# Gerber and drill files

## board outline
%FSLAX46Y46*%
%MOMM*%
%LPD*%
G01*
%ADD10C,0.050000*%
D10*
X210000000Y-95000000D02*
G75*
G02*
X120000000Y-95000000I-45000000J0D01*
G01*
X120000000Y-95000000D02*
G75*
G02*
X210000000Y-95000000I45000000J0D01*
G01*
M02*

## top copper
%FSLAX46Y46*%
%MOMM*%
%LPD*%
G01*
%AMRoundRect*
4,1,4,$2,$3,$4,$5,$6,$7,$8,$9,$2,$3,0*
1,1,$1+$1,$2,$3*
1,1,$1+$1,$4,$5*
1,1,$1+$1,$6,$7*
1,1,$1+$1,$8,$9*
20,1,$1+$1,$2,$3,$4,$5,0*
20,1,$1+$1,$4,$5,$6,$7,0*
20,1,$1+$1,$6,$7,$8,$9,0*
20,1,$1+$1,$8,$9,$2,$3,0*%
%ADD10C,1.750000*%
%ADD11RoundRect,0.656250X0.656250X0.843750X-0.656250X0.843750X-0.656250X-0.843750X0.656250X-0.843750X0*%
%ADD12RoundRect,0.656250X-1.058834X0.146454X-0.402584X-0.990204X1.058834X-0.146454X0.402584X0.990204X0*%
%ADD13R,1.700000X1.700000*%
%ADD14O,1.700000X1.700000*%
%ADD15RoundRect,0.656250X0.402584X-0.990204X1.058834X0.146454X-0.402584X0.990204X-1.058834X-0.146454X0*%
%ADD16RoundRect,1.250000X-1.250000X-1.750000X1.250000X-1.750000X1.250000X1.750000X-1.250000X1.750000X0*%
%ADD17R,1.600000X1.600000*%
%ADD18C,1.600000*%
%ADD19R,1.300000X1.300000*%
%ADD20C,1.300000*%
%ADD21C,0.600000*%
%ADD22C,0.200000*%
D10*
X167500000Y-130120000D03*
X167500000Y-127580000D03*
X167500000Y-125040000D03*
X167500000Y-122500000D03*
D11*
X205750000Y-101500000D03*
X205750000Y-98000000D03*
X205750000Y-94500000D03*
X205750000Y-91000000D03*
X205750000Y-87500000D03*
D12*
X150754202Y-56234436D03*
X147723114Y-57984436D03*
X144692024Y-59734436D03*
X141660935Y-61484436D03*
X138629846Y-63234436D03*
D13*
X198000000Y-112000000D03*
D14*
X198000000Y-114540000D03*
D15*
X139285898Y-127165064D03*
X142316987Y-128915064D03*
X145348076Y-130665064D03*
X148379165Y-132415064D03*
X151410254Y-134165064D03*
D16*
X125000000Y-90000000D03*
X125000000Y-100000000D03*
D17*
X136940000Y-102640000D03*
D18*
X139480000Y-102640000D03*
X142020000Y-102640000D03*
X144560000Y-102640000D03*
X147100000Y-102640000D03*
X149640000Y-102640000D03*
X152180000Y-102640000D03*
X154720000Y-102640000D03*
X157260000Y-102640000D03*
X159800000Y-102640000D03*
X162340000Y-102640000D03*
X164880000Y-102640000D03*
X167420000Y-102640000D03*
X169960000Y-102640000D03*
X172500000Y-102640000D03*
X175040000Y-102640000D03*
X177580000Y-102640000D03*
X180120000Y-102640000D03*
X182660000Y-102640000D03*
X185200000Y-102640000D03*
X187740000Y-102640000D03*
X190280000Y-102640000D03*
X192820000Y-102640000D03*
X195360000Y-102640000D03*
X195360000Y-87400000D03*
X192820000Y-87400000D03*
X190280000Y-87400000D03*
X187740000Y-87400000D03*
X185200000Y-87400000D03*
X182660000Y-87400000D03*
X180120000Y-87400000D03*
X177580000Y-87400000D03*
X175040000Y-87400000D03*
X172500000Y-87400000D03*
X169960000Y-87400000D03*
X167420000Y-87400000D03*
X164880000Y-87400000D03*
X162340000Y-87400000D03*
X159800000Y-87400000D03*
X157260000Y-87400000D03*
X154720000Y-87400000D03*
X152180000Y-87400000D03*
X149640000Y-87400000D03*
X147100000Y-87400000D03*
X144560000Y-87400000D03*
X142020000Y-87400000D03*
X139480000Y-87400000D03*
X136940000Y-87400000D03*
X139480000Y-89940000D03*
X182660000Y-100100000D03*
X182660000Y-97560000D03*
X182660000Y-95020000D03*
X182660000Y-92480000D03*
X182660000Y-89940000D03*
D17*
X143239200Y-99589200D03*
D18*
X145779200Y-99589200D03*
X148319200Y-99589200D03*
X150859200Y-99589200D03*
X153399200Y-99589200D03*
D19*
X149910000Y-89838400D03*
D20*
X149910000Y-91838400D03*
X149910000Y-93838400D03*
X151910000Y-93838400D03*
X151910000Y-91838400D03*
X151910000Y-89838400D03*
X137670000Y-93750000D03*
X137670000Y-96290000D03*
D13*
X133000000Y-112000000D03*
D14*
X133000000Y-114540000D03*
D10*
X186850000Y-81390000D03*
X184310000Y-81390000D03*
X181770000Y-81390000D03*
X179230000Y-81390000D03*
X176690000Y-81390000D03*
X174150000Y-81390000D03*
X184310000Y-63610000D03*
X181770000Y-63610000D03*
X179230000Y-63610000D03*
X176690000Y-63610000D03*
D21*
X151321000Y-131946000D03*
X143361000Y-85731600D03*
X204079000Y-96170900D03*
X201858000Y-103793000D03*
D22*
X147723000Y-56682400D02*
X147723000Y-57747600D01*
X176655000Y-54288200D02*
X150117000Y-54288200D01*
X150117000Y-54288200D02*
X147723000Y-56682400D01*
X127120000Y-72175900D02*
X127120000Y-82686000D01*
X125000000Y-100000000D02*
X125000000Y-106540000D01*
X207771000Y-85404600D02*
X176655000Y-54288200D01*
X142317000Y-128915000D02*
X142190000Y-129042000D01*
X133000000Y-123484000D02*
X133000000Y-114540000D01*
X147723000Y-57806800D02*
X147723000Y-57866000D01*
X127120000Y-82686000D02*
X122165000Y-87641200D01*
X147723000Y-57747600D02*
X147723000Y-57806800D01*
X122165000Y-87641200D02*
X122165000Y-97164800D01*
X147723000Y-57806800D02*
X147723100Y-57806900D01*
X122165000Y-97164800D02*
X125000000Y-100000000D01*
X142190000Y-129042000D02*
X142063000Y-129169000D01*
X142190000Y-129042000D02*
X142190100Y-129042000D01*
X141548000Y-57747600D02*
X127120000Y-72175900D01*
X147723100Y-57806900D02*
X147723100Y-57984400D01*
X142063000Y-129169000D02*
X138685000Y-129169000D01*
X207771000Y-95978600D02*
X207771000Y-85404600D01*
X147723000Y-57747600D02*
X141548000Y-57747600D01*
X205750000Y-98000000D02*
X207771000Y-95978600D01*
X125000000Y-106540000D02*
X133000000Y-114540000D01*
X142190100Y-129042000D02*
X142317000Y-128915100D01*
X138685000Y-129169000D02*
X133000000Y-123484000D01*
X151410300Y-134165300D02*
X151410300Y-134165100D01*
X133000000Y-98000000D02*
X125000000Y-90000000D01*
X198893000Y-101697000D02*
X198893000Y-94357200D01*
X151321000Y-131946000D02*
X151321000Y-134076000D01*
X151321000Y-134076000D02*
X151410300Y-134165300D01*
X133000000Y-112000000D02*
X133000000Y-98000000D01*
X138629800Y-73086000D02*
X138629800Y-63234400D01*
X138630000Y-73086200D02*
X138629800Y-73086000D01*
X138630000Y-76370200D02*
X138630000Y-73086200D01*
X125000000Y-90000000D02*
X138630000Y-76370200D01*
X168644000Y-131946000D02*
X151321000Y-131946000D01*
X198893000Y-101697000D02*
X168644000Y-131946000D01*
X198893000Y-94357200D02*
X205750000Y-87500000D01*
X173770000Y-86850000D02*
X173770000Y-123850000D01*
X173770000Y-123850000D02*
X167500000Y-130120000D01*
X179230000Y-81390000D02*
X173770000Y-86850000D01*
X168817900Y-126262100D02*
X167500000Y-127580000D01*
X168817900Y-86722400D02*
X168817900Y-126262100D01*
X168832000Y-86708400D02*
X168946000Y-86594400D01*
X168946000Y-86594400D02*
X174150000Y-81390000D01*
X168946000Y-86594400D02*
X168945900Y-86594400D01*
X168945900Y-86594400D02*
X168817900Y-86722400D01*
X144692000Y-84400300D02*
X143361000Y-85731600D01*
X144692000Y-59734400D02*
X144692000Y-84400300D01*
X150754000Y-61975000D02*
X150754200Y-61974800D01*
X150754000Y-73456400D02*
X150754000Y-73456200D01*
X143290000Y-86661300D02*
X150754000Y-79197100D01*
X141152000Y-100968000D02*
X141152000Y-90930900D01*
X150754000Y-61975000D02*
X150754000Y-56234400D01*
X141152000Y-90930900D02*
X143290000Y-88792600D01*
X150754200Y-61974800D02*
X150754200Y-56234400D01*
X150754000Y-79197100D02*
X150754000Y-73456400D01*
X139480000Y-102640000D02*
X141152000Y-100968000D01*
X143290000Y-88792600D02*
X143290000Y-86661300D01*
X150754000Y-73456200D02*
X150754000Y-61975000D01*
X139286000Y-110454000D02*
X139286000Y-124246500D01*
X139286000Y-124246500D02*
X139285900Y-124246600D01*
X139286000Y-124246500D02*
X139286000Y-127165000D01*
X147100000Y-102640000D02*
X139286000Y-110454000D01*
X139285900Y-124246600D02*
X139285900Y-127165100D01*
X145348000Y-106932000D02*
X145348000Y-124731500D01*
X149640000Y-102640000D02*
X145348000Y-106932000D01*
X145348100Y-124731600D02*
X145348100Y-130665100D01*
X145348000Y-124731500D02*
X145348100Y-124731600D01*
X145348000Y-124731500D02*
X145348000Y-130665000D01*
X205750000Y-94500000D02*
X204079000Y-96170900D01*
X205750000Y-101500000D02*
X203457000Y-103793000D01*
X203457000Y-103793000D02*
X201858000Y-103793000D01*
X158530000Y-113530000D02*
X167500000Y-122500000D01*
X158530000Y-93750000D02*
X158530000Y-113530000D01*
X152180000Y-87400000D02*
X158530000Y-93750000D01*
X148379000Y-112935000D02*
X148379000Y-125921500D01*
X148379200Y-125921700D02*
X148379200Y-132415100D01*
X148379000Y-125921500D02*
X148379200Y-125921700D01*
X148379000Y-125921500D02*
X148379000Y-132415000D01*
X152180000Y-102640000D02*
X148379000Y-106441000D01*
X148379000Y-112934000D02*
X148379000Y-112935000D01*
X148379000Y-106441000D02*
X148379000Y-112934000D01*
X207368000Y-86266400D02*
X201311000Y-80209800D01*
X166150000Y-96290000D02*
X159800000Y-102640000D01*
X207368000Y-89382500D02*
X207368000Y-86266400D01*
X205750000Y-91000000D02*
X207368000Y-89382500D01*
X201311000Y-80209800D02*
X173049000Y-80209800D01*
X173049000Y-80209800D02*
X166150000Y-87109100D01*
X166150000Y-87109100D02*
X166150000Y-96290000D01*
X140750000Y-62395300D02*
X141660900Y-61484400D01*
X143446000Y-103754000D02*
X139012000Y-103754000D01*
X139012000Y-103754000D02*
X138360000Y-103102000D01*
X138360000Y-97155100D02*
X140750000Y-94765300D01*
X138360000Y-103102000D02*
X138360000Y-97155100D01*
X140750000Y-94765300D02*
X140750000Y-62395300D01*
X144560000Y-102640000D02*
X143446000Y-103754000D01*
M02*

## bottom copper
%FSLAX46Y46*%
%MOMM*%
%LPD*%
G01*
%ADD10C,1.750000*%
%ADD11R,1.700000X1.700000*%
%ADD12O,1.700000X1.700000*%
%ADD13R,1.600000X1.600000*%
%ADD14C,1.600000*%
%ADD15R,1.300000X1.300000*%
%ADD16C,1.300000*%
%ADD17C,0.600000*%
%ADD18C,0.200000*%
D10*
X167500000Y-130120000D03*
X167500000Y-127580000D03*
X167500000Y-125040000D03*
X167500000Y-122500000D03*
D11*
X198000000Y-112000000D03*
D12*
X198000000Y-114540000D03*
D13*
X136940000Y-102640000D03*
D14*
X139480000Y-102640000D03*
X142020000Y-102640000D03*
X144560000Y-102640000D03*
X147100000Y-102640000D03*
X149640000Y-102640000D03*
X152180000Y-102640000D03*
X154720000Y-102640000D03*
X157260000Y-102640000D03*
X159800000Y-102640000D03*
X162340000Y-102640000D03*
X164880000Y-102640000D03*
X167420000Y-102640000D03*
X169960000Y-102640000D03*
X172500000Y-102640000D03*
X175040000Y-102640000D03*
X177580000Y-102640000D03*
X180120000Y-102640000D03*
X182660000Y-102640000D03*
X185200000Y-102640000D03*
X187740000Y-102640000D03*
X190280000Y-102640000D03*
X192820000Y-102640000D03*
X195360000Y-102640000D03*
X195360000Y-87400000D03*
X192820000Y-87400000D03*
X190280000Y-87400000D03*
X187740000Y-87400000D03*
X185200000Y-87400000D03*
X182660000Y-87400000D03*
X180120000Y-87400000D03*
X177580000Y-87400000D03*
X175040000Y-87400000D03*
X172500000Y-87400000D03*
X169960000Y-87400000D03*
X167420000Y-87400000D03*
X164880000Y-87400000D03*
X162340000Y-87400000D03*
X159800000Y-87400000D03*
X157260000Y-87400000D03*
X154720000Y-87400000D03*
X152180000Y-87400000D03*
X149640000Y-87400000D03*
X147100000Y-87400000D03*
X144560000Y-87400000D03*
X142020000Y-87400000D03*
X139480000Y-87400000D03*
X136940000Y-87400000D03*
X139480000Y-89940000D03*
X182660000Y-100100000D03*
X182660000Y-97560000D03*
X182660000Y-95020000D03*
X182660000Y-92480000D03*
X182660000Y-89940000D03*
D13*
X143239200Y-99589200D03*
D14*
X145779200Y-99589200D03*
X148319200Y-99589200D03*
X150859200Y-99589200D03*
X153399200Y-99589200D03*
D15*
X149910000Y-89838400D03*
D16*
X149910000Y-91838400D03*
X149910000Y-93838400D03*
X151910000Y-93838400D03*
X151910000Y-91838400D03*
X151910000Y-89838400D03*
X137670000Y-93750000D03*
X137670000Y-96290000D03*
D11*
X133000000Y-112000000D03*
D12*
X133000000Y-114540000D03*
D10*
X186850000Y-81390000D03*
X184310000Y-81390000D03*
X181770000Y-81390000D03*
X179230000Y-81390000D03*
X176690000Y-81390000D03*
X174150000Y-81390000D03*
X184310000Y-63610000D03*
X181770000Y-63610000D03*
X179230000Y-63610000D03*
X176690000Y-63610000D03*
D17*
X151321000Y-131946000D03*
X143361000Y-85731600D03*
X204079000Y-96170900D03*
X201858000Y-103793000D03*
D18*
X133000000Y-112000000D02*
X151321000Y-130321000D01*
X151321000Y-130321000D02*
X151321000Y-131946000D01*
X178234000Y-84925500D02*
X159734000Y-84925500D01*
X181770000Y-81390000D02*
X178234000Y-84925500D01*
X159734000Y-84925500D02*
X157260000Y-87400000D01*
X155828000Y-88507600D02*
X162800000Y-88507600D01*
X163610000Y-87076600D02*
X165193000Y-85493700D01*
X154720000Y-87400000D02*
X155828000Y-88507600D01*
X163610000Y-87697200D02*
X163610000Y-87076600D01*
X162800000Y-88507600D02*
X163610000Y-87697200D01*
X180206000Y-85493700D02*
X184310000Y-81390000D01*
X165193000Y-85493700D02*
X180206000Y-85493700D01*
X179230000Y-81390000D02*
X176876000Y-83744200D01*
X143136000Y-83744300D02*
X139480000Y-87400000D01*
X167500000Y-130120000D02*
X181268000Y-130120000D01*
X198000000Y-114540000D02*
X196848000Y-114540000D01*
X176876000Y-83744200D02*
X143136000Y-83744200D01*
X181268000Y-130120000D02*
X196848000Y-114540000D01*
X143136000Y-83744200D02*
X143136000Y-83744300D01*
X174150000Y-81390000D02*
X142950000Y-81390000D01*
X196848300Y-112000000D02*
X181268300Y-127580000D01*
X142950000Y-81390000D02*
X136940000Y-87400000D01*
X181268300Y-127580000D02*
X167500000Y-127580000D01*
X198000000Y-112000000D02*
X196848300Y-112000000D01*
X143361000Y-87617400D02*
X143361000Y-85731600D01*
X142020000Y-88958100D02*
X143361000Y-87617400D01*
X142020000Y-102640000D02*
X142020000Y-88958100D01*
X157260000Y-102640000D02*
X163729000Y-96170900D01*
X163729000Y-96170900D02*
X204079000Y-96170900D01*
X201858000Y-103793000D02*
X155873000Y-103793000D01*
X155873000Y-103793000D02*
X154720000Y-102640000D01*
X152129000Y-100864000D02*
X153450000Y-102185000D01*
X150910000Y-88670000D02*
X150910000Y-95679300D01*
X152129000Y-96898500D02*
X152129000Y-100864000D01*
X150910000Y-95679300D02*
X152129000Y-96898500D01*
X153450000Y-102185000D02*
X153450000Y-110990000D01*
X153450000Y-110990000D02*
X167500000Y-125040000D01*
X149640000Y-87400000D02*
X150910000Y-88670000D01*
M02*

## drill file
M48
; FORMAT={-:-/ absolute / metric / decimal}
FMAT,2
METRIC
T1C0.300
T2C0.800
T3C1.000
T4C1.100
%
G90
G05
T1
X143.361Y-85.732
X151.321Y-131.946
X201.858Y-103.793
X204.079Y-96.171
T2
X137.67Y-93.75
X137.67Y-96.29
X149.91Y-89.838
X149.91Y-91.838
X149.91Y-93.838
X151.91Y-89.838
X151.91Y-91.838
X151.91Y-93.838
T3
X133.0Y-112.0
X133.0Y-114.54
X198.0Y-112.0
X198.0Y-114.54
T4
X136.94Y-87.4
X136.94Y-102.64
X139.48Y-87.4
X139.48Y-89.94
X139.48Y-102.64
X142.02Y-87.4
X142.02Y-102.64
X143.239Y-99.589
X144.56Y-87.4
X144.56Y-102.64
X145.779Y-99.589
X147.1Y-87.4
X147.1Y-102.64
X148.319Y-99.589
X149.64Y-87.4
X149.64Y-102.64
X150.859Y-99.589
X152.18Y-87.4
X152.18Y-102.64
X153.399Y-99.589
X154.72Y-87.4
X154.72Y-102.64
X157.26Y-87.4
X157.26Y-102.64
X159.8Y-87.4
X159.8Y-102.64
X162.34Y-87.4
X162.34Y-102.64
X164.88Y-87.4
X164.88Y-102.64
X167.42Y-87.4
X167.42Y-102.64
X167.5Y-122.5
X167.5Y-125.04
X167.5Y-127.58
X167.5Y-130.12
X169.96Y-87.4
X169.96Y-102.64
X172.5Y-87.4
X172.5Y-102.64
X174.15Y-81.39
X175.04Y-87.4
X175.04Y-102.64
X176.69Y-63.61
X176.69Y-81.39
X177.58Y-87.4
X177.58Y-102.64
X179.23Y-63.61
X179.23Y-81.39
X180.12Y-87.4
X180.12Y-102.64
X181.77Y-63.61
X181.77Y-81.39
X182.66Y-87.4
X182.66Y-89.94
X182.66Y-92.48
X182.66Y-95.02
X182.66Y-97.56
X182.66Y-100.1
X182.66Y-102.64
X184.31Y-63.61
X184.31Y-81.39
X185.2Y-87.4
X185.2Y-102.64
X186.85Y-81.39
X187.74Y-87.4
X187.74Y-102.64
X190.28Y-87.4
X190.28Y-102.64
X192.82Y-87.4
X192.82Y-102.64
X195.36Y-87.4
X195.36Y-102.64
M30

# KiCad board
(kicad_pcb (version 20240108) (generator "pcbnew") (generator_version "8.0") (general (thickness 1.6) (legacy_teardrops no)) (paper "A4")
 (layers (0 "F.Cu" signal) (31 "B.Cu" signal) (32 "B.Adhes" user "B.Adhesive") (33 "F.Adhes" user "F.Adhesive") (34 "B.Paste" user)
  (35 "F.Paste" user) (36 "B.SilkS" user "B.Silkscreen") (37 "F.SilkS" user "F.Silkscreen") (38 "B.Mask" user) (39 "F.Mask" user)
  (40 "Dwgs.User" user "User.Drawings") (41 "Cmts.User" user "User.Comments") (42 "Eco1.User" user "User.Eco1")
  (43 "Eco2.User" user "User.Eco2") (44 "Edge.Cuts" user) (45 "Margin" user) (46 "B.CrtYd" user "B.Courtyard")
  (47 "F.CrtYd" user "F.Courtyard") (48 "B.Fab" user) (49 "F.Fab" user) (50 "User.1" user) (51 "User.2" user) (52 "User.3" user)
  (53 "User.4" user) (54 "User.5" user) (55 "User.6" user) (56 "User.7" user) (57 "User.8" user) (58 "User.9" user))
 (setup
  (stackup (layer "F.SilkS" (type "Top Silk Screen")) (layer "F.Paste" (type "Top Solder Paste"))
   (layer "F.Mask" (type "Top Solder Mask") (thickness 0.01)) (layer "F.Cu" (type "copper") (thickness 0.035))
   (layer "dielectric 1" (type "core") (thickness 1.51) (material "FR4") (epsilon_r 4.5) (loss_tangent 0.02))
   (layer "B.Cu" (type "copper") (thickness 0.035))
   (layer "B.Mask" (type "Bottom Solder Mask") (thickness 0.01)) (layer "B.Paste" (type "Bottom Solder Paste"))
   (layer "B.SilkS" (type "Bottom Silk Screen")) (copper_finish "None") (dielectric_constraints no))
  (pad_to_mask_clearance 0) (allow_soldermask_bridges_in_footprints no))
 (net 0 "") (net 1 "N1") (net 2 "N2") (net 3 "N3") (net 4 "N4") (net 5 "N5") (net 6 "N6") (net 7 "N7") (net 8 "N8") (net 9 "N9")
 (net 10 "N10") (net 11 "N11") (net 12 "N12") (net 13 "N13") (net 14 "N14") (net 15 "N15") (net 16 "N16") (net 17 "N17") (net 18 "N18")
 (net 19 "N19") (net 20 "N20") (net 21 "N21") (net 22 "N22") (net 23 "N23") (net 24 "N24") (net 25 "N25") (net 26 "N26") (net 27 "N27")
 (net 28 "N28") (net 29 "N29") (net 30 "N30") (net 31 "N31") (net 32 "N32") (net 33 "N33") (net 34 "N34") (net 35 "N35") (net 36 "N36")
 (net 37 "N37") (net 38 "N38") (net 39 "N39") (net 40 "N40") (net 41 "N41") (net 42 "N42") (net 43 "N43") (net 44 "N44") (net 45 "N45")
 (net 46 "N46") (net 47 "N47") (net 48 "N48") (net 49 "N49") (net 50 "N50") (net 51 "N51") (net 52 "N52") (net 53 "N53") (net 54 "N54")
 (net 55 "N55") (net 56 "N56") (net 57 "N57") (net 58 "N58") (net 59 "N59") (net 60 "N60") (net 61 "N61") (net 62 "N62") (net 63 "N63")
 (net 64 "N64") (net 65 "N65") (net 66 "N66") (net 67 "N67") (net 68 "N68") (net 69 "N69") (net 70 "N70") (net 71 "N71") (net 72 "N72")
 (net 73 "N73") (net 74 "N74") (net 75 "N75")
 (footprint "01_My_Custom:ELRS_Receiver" (layer "F.Cu") (at 181.2 126.31)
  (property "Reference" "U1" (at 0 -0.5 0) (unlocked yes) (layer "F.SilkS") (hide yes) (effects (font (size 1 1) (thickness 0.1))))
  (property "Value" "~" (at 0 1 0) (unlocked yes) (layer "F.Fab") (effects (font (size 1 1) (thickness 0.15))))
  (pad "1" thru_hole circle (at -13.7 3.81) (size 1.75 1.75) (drill 1.1) (layers "*.Cu" "*.Mask") (remove_unused_layers no) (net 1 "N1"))
  (pad "2" thru_hole circle (at -13.7 1.27) (size 1.75 1.75) (drill 1.1) (layers "*.Cu" "*.Mask") (remove_unused_layers no) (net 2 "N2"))
  (pad "3" thru_hole circle (at -13.7 -1.27) (size 1.75 1.75) (drill 1.1) (layers "*.Cu" "*.Mask") (remove_unused_layers no) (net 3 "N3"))
  (pad "4" thru_hole circle (at -13.7 -3.81) (size 1.75 1.75) (drill 1.1) (layers "*.Cu" "*.Mask") (remove_unused_layers no) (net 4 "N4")))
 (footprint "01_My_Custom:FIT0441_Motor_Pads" (layer "F.Cu") (at 203.25 97.5 180)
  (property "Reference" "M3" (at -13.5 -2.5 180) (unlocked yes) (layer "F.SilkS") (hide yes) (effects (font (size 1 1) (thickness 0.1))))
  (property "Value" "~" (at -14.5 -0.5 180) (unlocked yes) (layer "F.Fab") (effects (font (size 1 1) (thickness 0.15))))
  (pad "1" smd roundrect (at -2.5 -4 180) (size 2.625 3) (layers "F.Cu" "F.Paste" "F.Mask") (roundrect_rratio 0.25) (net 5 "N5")
   (thermal_bridge_angle 45))
  (pad "2" smd roundrect (at -2.5 -0.5 180) (size 2.625 3) (layers "F.Cu" "F.Paste" "F.Mask") (roundrect_rratio 0.25) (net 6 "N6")
   (thermal_bridge_angle 45))
  (pad "3" smd roundrect (at -2.5 3 180) (size 2.625 3) (layers "F.Cu" "F.Paste" "F.Mask") (roundrect_rratio 0.25) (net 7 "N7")
   (thermal_bridge_angle 45))
  (pad "4" smd roundrect (at -2.5 6.5 180) (size 2.625 3) (layers "F.Cu" "F.Paste" "F.Mask") (roundrect_rratio 0.25) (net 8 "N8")
   (thermal_bridge_angle 45))
  (pad "5" smd roundrect (at -2.5 10 180) (size 2.625 3) (layers "F.Cu" "F.Paste" "F.Mask") (roundrect_rratio 0.25) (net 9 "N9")
   (thermal_bridge_angle 45)))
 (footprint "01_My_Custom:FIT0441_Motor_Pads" (layer "F.Cu") (at 148.5401 60.3995 -60)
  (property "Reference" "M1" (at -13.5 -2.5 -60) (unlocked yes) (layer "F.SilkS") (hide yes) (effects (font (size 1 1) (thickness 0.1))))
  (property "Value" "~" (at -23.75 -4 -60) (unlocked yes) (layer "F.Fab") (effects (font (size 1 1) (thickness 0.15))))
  (pad "1" smd roundrect (at -2.5 -4.000001 300) (size 2.625 3) (layers "F.Cu" "F.Paste" "F.Mask") (roundrect_rratio 0.25) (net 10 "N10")
   (thermal_bridge_angle 45))
  (pad "2" smd roundrect (at -2.5 -0.500001 300) (size 2.625 3) (layers "F.Cu" "F.Paste" "F.Mask") (roundrect_rratio 0.25) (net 6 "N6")
   (thermal_bridge_angle 45))
  (pad "3" smd roundrect (at -2.5 3 300) (size 2.625 3) (layers "F.Cu" "F.Paste" "F.Mask") (roundrect_rratio 0.25) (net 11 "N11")
   (thermal_bridge_angle 45))
  (pad "4" smd roundrect (at -2.5 6.5 300) (size 2.625 3) (layers "F.Cu" "F.Paste" "F.Mask") (roundrect_rratio 0.25) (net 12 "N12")
   (thermal_bridge_angle 45))
  (pad "5" smd roundrect (at -2.5 10 300) (size 2.625 3) (layers "F.Cu" "F.Paste" "F.Mask") (roundrect_rratio 0.25) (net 9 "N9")
   (thermal_bridge_angle 45)))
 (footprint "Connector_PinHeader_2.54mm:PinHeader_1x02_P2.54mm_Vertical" (layer "F.Cu") (at 198 112)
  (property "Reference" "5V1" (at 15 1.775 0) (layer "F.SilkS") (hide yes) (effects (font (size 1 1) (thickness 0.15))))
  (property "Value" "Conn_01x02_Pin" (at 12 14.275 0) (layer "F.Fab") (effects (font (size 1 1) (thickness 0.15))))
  (pad "1" thru_hole rect (at 0 0) (size 1.7 1.7) (drill 1) (layers "*.Cu" "*.Mask") (remove_unused_layers no) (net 2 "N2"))
  (pad "2" thru_hole oval (at 0 2.54) (size 1.7 1.7) (drill 1) (layers "*.Cu" "*.Mask") (remove_unused_layers no) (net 1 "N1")))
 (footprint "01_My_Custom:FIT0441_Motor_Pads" (layer "F.Cu") (at 144 127 60)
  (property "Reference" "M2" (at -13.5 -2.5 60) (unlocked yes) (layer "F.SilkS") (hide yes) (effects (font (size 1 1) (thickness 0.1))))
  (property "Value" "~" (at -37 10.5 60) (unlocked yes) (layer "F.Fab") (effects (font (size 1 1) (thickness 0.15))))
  (pad "1" smd roundrect (at -2.500001 -4 60) (size 2.625 3) (layers "F.Cu" "F.Paste" "F.Mask") (roundrect_rratio 0.25) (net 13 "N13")
   (thermal_bridge_angle 45))
  (pad "2" smd roundrect (at -2.500001 -0.5 60) (size 2.625 3) (layers "F.Cu" "F.Paste" "F.Mask") (roundrect_rratio 0.25) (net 6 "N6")
   (thermal_bridge_angle 45))
  (pad "3" smd roundrect (at -2.500001 3 60) (size 2.625 3) (layers "F.Cu" "F.Paste" "F.Mask") (roundrect_rratio 0.25) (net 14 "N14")
   (thermal_bridge_angle 45))
  (pad "4" smd roundrect (at -2.5 6.5 60) (size 2.625 3) (layers "F.Cu" "F.Paste" "F.Mask") (roundrect_rratio 0.25) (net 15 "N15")
   (thermal_bridge_angle 45))
  (pad "5" smd roundrect (at -2.5 10 60) (size 2.625 3) (layers "F.Cu" "F.Paste" "F.Mask") (roundrect_rratio 0.25) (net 9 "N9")
   (thermal_bridge_angle 45)))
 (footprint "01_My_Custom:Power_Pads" (layer "F.Cu") (at 125 95)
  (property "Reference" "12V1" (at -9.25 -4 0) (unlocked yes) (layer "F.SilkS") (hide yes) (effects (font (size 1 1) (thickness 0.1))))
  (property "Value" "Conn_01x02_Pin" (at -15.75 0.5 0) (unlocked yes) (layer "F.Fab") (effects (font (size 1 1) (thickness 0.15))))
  (pad "1" smd roundrect (at 0 -5) (size 5 6) (layers "F.Cu" "F.Paste" "F.Mask") (roundrect_rratio 0.25) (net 9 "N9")
   (thermal_bridge_angle 45))
  (pad "2" smd roundrect (at 0 5) (size 5 6) (layers "F.Cu" "F.Paste" "F.Mask") (roundrect_rratio 0.25) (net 6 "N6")
   (thermal_bridge_angle 45)))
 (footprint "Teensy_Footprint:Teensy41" (layer "F.Cu") (at 166.15 95.02)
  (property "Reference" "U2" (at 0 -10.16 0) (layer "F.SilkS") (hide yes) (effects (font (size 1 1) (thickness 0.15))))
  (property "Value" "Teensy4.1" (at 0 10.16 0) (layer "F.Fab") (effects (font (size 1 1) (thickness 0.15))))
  (pad "1" thru_hole rect (at -29.21 7.62) (size 1.6 1.6) (drill 1.1) (layers "*.Cu" "*.Mask") (remove_unused_layers no) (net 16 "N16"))
  (pad "2" thru_hole circle (at -26.67 7.62) (size 1.6 1.6) (drill 1.1) (layers "*.Cu" "*.Mask") (remove_unused_layers no) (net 10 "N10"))
  (pad "3" thru_hole circle (at -24.13 7.62) (size 1.6 1.6) (drill 1.1) (layers "*.Cu" "*.Mask") (remove_unused_layers no) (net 11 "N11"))
  (pad "4" thru_hole circle (at -21.59 7.62) (size 1.6 1.6) (drill 1.1) (layers "*.Cu" "*.Mask") (remove_unused_layers no) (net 12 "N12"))
  (pad "5" thru_hole circle (at -19.05 7.62) (size 1.6 1.6) (drill 1.1) (layers "*.Cu" "*.Mask") (remove_unused_layers no) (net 13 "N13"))
  (pad "6" thru_hole circle (at -16.51 7.62) (size 1.6 1.6) (drill 1.1) (layers "*.Cu" "*.Mask") (remove_unused_layers no) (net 14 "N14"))
  (pad "7" thru_hole circle (at -13.97 7.62) (size 1.6 1.6) (drill 1.1) (layers "*.Cu" "*.Mask") (remove_unused_layers no) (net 15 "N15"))
  (pad "8" thru_hole circle (at -11.43 7.62) (size 1.6 1.6) (drill 1.1) (layers "*.Cu" "*.Mask") (remove_unused_layers no) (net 5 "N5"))
  (pad "9" thru_hole circle (at -8.89 7.62) (size 1.6 1.6) (drill 1.1) (layers "*.Cu" "*.Mask") (remove_unused_layers no) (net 7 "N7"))
  (pad "10" thru_hole circle (at -6.35 7.62) (size 1.6 1.6) (drill 1.1) (layers "*.Cu" "*.Mask") (remove_unused_layers no) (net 8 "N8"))
  (pad "11" thru_hole circle (at -3.81 7.62) (size 1.6 1.6) (drill 1.1) (layers "*.Cu" "*.Mask") (remove_unused_layers no) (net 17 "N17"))
  (pad "12" thru_hole circle (at -1.27 7.62) (size 1.6 1.6) (drill 1.1) (layers "*.Cu" "*.Mask") (remove_unused_layers no) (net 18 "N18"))
  (pad "13" thru_hole circle (at 1.27 7.62) (size 1.6 1.6) (drill 1.1) (layers "*.Cu" "*.Mask") (remove_unused_layers no) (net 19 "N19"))
  (pad "14" thru_hole circle (at 3.81 7.62) (size 1.6 1.6) (drill 1.1) (layers "*.Cu" "*.Mask") (remove_unused_layers no) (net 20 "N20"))
  (pad "15" thru_hole circle (at 6.35 7.62) (size 1.6 1.6) (drill 1.1) (layers "*.Cu" "*.Mask") (remove_unused_layers no) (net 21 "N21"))
  (pad "16" thru_hole circle (at 8.89 7.62) (size 1.6 1.6) (drill 1.1) (layers "*.Cu" "*.Mask") (remove_unused_layers no) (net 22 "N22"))
  (pad "17" thru_hole circle (at 11.43 7.62) (size 1.6 1.6) (drill 1.1) (layers "*.Cu" "*.Mask") (remove_unused_layers no) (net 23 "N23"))
  (pad "18" thru_hole circle (at 13.97 7.62) (size 1.6 1.6) (drill 1.1) (layers "*.Cu" "*.Mask") (remove_unused_layers no) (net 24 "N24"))
  (pad "19" thru_hole circle (at 16.51 7.62) (size 1.6 1.6) (drill 1.1) (layers "*.Cu" "*.Mask") (remove_unused_layers no) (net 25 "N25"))
  (pad "20" thru_hole circle (at 19.05 7.62) (size 1.6 1.6) (drill 1.1) (layers "*.Cu" "*.Mask") (remove_unused_layers no) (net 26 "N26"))
  (pad "21" thru_hole circle (at 21.59 7.62) (size 1.6 1.6) (drill 1.1) (layers "*.Cu" "*.Mask") (remove_unused_layers no) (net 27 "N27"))
  (pad "22" thru_hole circle (at 24.13 7.62) (size 1.6 1.6) (drill 1.1) (layers "*.Cu" "*.Mask") (remove_unused_layers no) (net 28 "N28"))
  (pad "23" thru_hole circle (at 26.67 7.62) (size 1.6 1.6) (drill 1.1) (layers "*.Cu" "*.Mask") (remove_unused_layers no) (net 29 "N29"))
  (pad "24" thru_hole circle (at 29.21 7.62) (size 1.6 1.6) (drill 1.1) (layers "*.Cu" "*.Mask") (remove_unused_layers no) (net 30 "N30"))
  (pad "25" thru_hole circle (at 29.21 -7.62) (size 1.6 1.6) (drill 1.1) (layers "*.Cu" "*.Mask") (remove_unused_layers no) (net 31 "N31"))
  (pad "26" thru_hole circle (at 26.67 -7.62) (size 1.6 1.6) (drill 1.1) (layers "*.Cu" "*.Mask") (remove_unused_layers no) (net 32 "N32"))
  (pad "27" thru_hole circle (at 24.13 -7.62) (size 1.6 1.6) (drill 1.1) (layers "*.Cu" "*.Mask") (remove_unused_layers no) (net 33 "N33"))
  (pad "28" thru_hole circle (at 21.59 -7.62) (size 1.6 1.6) (drill 1.1) (layers "*.Cu" "*.Mask") (remove_unused_layers no) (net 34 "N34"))
  (pad "29" thru_hole circle (at 19.05 -7.62) (size 1.6 1.6) (drill 1.1) (layers "*.Cu" "*.Mask") (remove_unused_layers no) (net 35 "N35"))
  (pad "30" thru_hole circle (at 16.51 -7.62) (size 1.6 1.6) (drill 1.1) (layers "*.Cu" "*.Mask") (remove_unused_layers no) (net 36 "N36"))
  (pad "31" thru_hole circle (at 13.97 -7.62) (size 1.6 1.6) (drill 1.1) (layers "*.Cu" "*.Mask") (remove_unused_layers no) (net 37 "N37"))
  (pad "32" thru_hole circle (at 11.43 -7.62) (size 1.6 1.6) (drill 1.1) (layers "*.Cu" "*.Mask") (remove_unused_layers no) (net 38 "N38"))
  (pad "33" thru_hole circle (at 8.89 -7.62) (size 1.6 1.6) (drill 1.1) (layers "*.Cu" "*.Mask") (remove_unused_layers no) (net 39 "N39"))
  (pad "34" thru_hole circle (at 6.35 -7.62) (size 1.6 1.6) (drill 1.1) (layers "*.Cu" "*.Mask") (remove_unused_layers no) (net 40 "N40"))
  (pad "35" thru_hole circle (at 3.81 -7.62) (size 1.6 1.6) (drill 1.1) (layers "*.Cu" "*.Mask") (remove_unused_layers no) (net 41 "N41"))
  (pad "36" thru_hole circle (at 1.27 -7.62) (size 1.6 1.6) (drill 1.1) (layers "*.Cu" "*.Mask") (remove_unused_layers no) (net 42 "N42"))
  (pad "37" thru_hole circle (at -1.27 -7.62) (size 1.6 1.6) (drill 1.1) (layers "*.Cu" "*.Mask") (remove_unused_layers no) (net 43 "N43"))
  (pad "38" thru_hole circle (at -3.81 -7.62) (size 1.6 1.6) (drill 1.1) (layers "*.Cu" "*.Mask") (remove_unused_layers no) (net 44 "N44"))
  (pad "39" thru_hole circle (at -6.35 -7.62) (size 1.6 1.6) (drill 1.1) (layers "*.Cu" "*.Mask") (remove_unused_layers no) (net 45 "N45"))
  (pad "40" thru_hole circle (at -8.89 -7.62) (size 1.6 1.6) (drill 1.1) (layers "*.Cu" "*.Mask") (remove_unused_layers no) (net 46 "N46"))
  (pad "41" thru_hole circle (at -11.43 -7.62) (size 1.6 1.6) (drill 1.1) (layers "*.Cu" "*.Mask") (remove_unused_layers no) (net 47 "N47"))
  (pad "42" thru_hole circle (at -13.97 -7.62) (size 1.6 1.6) (drill 1.1) (layers "*.Cu" "*.Mask") (remove_unused_layers no) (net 4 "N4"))
  (pad "43" thru_hole circle (at -16.51 -7.62) (size 1.6 1.6) (drill 1.1) (layers "*.Cu" "*.Mask") (remove_unused_layers no) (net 3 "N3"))
  (pad "44" thru_hole circle (at -19.05 -7.62) (size 1.6 1.6) (drill 1.1) (layers "*.Cu" "*.Mask") (remove_unused_layers no) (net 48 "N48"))
  (pad "45" thru_hole circle (at -21.59 -7.62) (size 1.6 1.6) (drill 1.1) (layers "*.Cu" "*.Mask") (remove_unused_layers no) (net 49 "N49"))
  (pad "46" thru_hole circle (at -24.13 -7.62) (size 1.6 1.6) (drill 1.1) (layers "*.Cu" "*.Mask") (remove_unused_layers no) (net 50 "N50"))
  (pad "47" thru_hole circle (at -26.67 -7.62) (size 1.6 1.6) (drill 1.1) (layers "*.Cu" "*.Mask") (remove_unused_layers no) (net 1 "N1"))
  (pad "48" thru_hole circle (at -29.21 -7.62) (size 1.6 1.6) (drill 1.1) (layers "*.Cu" "*.Mask") (remove_unused_layers no) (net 2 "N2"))
  (pad "49" thru_hole circle (at -26.67 -5.08) (size 1.6 1.6) (drill 1.1) (layers "*.Cu" "*.Mask") (remove_unused_layers no) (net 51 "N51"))
  (pad "50" thru_hole circle (at 16.51 5.08) (size 1.6 1.6) (drill 1.1) (layers "*.Cu" "*.Mask") (remove_unused_layers no) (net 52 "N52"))
  (pad "51" thru_hole circle (at 16.51 2.54) (size 1.6 1.6) (drill 1.1) (layers "*.Cu" "*.Mask") (remove_unused_layers no) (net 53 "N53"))
  (pad "52" thru_hole circle (at 16.51 0) (size 1.6 1.6) (drill 1.1) (layers "*.Cu" "*.Mask") (remove_unused_layers no) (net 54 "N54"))
  (pad "53" thru_hole circle (at 16.51 -2.54) (size 1.6 1.6) (drill 1.1) (layers "*.Cu" "*.Mask") (remove_unused_layers no) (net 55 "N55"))
  (pad "54" thru_hole circle (at 16.51 -5.08) (size 1.6 1.6) (drill 1.1) (layers "*.Cu" "*.Mask") (remove_unused_layers no) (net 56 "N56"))
  (pad "55" thru_hole rect (at -22.9108 4.5692) (size 1.6 1.6) (drill 1.1) (layers "*.Cu" "*.Mask") (remove_unused_layers no) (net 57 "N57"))
  (pad "56" thru_hole circle (at -20.3708 4.5692) (size 1.6 1.6) (drill 1.1) (layers "*.Cu" "*.Mask") (remove_unused_layers no)
   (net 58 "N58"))
  (pad "57" thru_hole circle (at -17.8308 4.5692) (size 1.6 1.6) (drill 1.1) (layers "*.Cu" "*.Mask") (remove_unused_layers no)
   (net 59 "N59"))
  (pad "58" thru_hole circle (at -15.2908 4.5692) (size 1.6 1.6) (drill 1.1) (layers "*.Cu" "*.Mask") (remove_unused_layers no)
   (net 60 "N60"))
  (pad "59" thru_hole circle (at -12.7508 4.5692) (size 1.6 1.6) (drill 1.1) (layers "*.Cu" "*.Mask") (remove_unused_layers no)
   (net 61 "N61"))
  (pad "60" thru_hole rect (at -16.24 -5.1816) (size 1.3 1.3) (drill 0.8) (layers "*.Cu" "*.Mask") (remove_unused_layers no) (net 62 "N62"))
  (pad "61" thru_hole circle (at -16.24 -3.1816) (size 1.3 1.3) (drill 0.8) (layers "*.Cu" "*.Mask") (remove_unused_layers no)
   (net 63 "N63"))
  (pad "62" thru_hole circle (at -16.24 -1.1816) (size 1.3 1.3) (drill 0.8) (layers "*.Cu" "*.Mask") (remove_unused_layers no)
   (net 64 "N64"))
  (pad "63" thru_hole circle (at -14.24 -1.1816) (size 1.3 1.3) (drill 0.8) (layers "*.Cu" "*.Mask") (remove_unused_layers no)
   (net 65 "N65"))
  (pad "64" thru_hole circle (at -14.24 -3.1816) (size 1.3 1.3) (drill 0.8) (layers "*.Cu" "*.Mask") (remove_unused_layers no)
   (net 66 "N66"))
  (pad "65" thru_hole circle (at -14.24 -5.1816) (size 1.3 1.3) (drill 0.8) (layers "*.Cu" "*.Mask") (remove_unused_layers no)
   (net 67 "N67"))
  (pad "66" thru_hole circle (at -28.48 -1.27) (size 1.3 1.3) (drill 0.8) (layers "*.Cu" "*.Mask") (remove_unused_layers no) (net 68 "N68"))
  (pad "67" thru_hole circle (at -28.48 1.27) (size 1.3 1.3) (drill 0.8) (layers "*.Cu" "*.Mask") (remove_unused_layers no) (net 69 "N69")))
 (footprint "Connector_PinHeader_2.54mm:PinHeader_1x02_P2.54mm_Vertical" (layer "F.Cu") (at 133 112)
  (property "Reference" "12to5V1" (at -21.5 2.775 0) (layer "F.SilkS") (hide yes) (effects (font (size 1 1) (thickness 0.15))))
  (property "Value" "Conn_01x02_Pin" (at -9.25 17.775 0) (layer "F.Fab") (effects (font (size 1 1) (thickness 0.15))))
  (pad "1" thru_hole rect (at 0 0) (size 1.7 1.7) (drill 1) (layers "*.Cu" "*.Mask") (remove_unused_layers no) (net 9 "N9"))
  (pad "2" thru_hole oval (at 0 2.54) (size 1.7 1.7) (drill 1) (layers "*.Cu" "*.Mask") (remove_unused_layers no) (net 6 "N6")))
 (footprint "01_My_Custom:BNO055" (layer "F.Cu") (at 180.5 72.5 -90)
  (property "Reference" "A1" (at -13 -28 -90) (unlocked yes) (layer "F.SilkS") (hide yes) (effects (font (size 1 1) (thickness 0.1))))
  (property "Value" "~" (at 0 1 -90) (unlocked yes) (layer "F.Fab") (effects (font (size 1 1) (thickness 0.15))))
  (pad "1" thru_hole circle (at 8.89 -6.35 270) (size 1.75 1.75) (drill 1.1) (layers "*.Cu" "*.Mask") (remove_unused_layers no)
   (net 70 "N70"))
  (pad "2" thru_hole circle (at 8.89 -3.81 270) (size 1.75 1.75) (drill 1.1) (layers "*.Cu" "*.Mask") (remove_unused_layers no)
   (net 47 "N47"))
  (pad "3" thru_hole circle (at 8.89 -1.27 270) (size 1.75 1.75) (drill 1.1) (layers "*.Cu" "*.Mask") (remove_unused_layers no)
   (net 46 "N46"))
  (pad "4" thru_hole circle (at 8.89 1.27 270) (size 1.75 1.75) (drill 1.1) (layers "*.Cu" "*.Mask") (remove_unused_layers no) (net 1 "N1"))
  (pad "5" thru_hole circle (at 8.89 3.81 270) (size 1.75 1.75) (drill 1.1) (layers "*.Cu" "*.Mask") (remove_unused_layers no)
   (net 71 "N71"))
  (pad "6" thru_hole circle (at 8.89 6.35 270) (size 1.75 1.75) (drill 1.1) (layers "*.Cu" "*.Mask") (remove_unused_layers no) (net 2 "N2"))
  (pad "7" thru_hole circle (at -8.89 -3.81 270) (size 1.75 1.75) (drill 1.1) (layers "*.Cu" "*.Mask") (remove_unused_layers no)
   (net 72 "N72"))
  (pad "8" thru_hole circle (at -8.89 -1.27 270) (size 1.75 1.75) (drill 1.1) (layers "*.Cu" "*.Mask") (remove_unused_layers no)
   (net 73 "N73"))
  (pad "9" thru_hole circle (at -8.89 1.27 270) (size 1.75 1.75) (drill 1.1) (layers "*.Cu" "*.Mask") (remove_unused_layers no)
   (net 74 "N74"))
  (pad "10" thru_hole circle (at -8.89 3.81 270) (size 1.75 1.75) (drill 1.1) (layers "*.Cu" "*.Mask") (remove_unused_layers no)
   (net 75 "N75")))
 (gr_circle (center 165 95) (end 210 95) (stroke (width 0.05) (type default)) (fill none) (layer "Edge.Cuts"))
 (segment (start 147.723 56.6824) (end 147.723 57.7476) (width 0.2) (layer "F.Cu") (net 6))
 (segment (start 176.655 54.2882) (end 150.117 54.2882) (width 0.2) (layer "F.Cu") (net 6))
 (segment (start 150.117 54.2882) (end 147.723 56.6824) (width 0.2) (layer "F.Cu") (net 6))
 (segment (start 127.12 72.1759) (end 127.12 82.686) (width 0.2) (layer "F.Cu") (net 6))
 (segment (start 125 100) (end 125 106.54) (width 0.2) (layer "F.Cu") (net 6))
 (segment (start 207.771 85.4046) (end 176.655 54.2882) (width 0.2) (layer "F.Cu") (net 6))
 (segment (start 142.317 128.915) (end 142.19 129.042) (width 0.2) (layer "F.Cu") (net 6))
 (segment (start 133 123.484) (end 133 114.54) (width 0.2) (layer "F.Cu") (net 6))
 (segment (start 147.723 57.8068) (end 147.723 57.866) (width 0.2) (layer "F.Cu") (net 6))
 (segment (start 127.12 82.686) (end 122.165 87.6412) (width 0.2) (layer "F.Cu") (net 6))
 (segment (start 147.723 57.7476) (end 147.723 57.8068) (width 0.2) (layer "F.Cu") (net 6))
 (segment (start 122.165 87.6412) (end 122.165 97.1648) (width 0.2) (layer "F.Cu") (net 6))
 (segment (start 147.723 57.8068) (end 147.7231 57.8069) (width 0.2) (layer "F.Cu") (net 6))
 (segment (start 122.165 97.1648) (end 125 100) (width 0.2) (layer "F.Cu") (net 6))
 (segment (start 142.19 129.042) (end 142.063 129.169) (width 0.2) (layer "F.Cu") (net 6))
 (segment (start 142.19 129.042) (end 142.1901 129.042) (width 0.2) (layer "F.Cu") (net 6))
 (segment (start 141.548 57.7476) (end 127.12 72.1759) (width 0.2) (layer "F.Cu") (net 6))
 (segment (start 147.7231 57.8069) (end 147.7231 57.9844) (width 0.2) (layer "F.Cu") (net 6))
 (segment (start 142.063 129.169) (end 138.685 129.169) (width 0.2) (layer "F.Cu") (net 6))
 (segment (start 207.771 95.9786) (end 207.771 85.4046) (width 0.2) (layer "F.Cu") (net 6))
 (segment (start 147.723 57.7476) (end 141.548 57.7476) (width 0.2) (layer "F.Cu") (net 6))
 (segment (start 205.75 98) (end 207.771 95.9786) (width 0.2) (layer "F.Cu") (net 6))
 (segment (start 125 106.54) (end 133 114.54) (width 0.2) (layer "F.Cu") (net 6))
 (segment (start 142.1901 129.042) (end 142.317 128.9151) (width 0.2) (layer "F.Cu") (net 6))
 (segment (start 138.685 129.169) (end 133 123.484) (width 0.2) (layer "F.Cu") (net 6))
 (segment (start 151.4103 134.1653) (end 151.4103 134.1651) (width 0.2) (layer "F.Cu") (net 9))
 (segment (start 133 98) (end 125 90) (width 0.2) (layer "F.Cu") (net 9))
 (segment (start 198.893 101.697) (end 198.893 94.3572) (width 0.2) (layer "F.Cu") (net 9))
 (segment (start 151.321 131.946) (end 151.321 134.076) (width 0.2) (layer "F.Cu") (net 9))
 (segment (start 151.321 134.076) (end 151.4103 134.1653) (width 0.2) (layer "F.Cu") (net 9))
 (segment (start 133 112) (end 133 98) (width 0.2) (layer "F.Cu") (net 9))
 (segment (start 138.6298 73.086) (end 138.6298 63.2344) (width 0.2) (layer "F.Cu") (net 9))
 (segment (start 138.63 73.0862) (end 138.6298 73.086) (width 0.2) (layer "F.Cu") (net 9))
 (segment (start 138.63 76.3702) (end 138.63 73.0862) (width 0.2) (layer "F.Cu") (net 9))
 (segment (start 125 90) (end 138.63 76.3702) (width 0.2) (layer "F.Cu") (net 9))
 (segment (start 168.644 131.946) (end 151.321 131.946) (width 0.2) (layer "F.Cu") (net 9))
 (segment (start 198.893 101.697) (end 168.644 131.946) (width 0.2) (layer "F.Cu") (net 9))
 (segment (start 198.893 94.3572) (end 205.75 87.5) (width 0.2) (layer "F.Cu") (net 9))
 (via (at 151.321 131.946) (size 0.6) (drill 0.3) (layers "F.Cu" "B.Cu") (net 9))
 (segment (start 133 112) (end 151.321 130.321) (width 0.2) (layer "B.Cu") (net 9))
 (segment (start 151.321 130.321) (end 151.321 131.946) (width 0.2) (layer "B.Cu") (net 9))
 (segment (start 178.234 84.9255) (end 159.734 84.9255) (width 0.2) (layer "B.Cu") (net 46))
 (segment (start 181.77 81.39) (end 178.234 84.9255) (width 0.2) (layer "B.Cu") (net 46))
 (segment (start 159.734 84.9255) (end 157.26 87.4) (width 0.2) (layer "B.Cu") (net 46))
 (segment (start 155.828 88.5076) (end 162.8 88.5076) (width 0.2) (layer "B.Cu") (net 47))
 (segment (start 163.61 87.0766) (end 165.193 85.4937) (width 0.2) (layer "B.Cu") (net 47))
 (segment (start 154.72 87.4) (end 155.828 88.5076) (width 0.2) (layer "B.Cu") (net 47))
 (segment (start 163.61 87.6972) (end 163.61 87.0766) (width 0.2) (layer "B.Cu") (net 47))
 (segment (start 162.8 88.5076) (end 163.61 87.6972) (width 0.2) (layer "B.Cu") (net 47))
 (segment (start 180.206 85.4937) (end 184.31 81.39) (width 0.2) (layer "B.Cu") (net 47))
 (segment (start 165.193 85.4937) (end 180.206 85.4937) (width 0.2) (layer "B.Cu") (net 47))
 (segment (start 173.77 86.85) (end 173.77 123.85) (width 0.2) (layer "F.Cu") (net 1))
 (segment (start 173.77 123.85) (end 167.5 130.12) (width 0.2) (layer "F.Cu") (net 1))
 (segment (start 179.23 81.39) (end 173.77 86.85) (width 0.2) (layer "F.Cu") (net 1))
 (segment (start 179.23 81.39) (end 176.876 83.7442) (width 0.2) (layer "B.Cu") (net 1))
 (segment (start 143.136 83.7443) (end 139.48 87.4) (width 0.2) (layer "B.Cu") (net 1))
 (segment (start 167.5 130.12) (end 181.268 130.12) (width 0.2) (layer "B.Cu") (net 1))
 (segment (start 198 114.54) (end 196.848 114.54) (width 0.2) (layer "B.Cu") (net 1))
 (segment (start 176.876 83.7442) (end 143.136 83.7442) (width 0.2) (layer "B.Cu") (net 1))
 (segment (start 181.268 130.12) (end 196.848 114.54) (width 0.2) (layer "B.Cu") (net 1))
 (segment (start 143.136 83.7442) (end 143.136 83.7443) (width 0.2) (layer "B.Cu") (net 1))
 (segment (start 168.8179 126.2621) (end 167.5 127.58) (width 0.2) (layer "F.Cu") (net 2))
 (segment (start 168.8179 86.7224) (end 168.8179 126.2621) (width 0.2) (layer "F.Cu") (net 2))
 (segment (start 168.832 86.7084) (end 168.946 86.5944) (width 0.2) (layer "F.Cu") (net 2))
 (segment (start 168.946 86.5944) (end 174.15 81.39) (width 0.2) (layer "F.Cu") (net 2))
 (segment (start 168.946 86.5944) (end 168.9459 86.5944) (width 0.2) (layer "F.Cu") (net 2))
 (segment (start 168.9459 86.5944) (end 168.8179 86.7224) (width 0.2) (layer "F.Cu") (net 2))
 (segment (start 174.15 81.39) (end 142.95 81.39) (width 0.2) (layer "B.Cu") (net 2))
 (segment (start 196.8483 112) (end 181.2683 127.58) (width 0.2) (layer "B.Cu") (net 2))
 (segment (start 142.95 81.39) (end 136.94 87.4) (width 0.2) (layer "B.Cu") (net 2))
 (segment (start 181.2683 127.58) (end 167.5 127.58) (width 0.2) (layer "B.Cu") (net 2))
 (segment (start 198 112) (end 196.8483 112) (width 0.2) (layer "B.Cu") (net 2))
 (segment (start 144.692 84.4003) (end 143.361 85.7316) (width 0.2) (layer "F.Cu") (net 11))
 (segment (start 144.692 59.7344) (end 144.692 84.4003) (width 0.2) (layer "F.Cu") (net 11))
 (via (at 143.361 85.7316) (size 0.6) (drill 0.3) (layers "F.Cu" "B.Cu") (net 11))
 (segment (start 143.361 87.6174) (end 143.361 85.7316) (width 0.2) (layer "B.Cu") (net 11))
 (segment (start 142.02 88.9581) (end 143.361 87.6174) (width 0.2) (layer "B.Cu") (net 11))
 (segment (start 142.02 102.64) (end 142.02 88.9581) (width 0.2) (layer "B.Cu") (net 11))
 (segment (start 150.754 61.975) (end 150.7542 61.9748) (width 0.2) (layer "F.Cu") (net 10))
 (segment (start 150.754 73.4564) (end 150.754 73.4562) (width 0.2) (layer "F.Cu") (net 10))
 (segment (start 143.29 86.6613) (end 150.754 79.1971) (width 0.2) (layer "F.Cu") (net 10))
 (segment (start 141.152 100.968) (end 141.152 90.9309) (width 0.2) (layer "F.Cu") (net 10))
 (segment (start 150.754 61.975) (end 150.754 56.2344) (width 0.2) (layer "F.Cu") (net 10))
 (segment (start 141.152 90.9309) (end 143.29 88.7926) (width 0.2) (layer "F.Cu") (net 10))
 (segment (start 150.7542 61.9748) (end 150.7542 56.2344) (width 0.2) (layer "F.Cu") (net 10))
 (segment (start 150.754 79.1971) (end 150.754 73.4564) (width 0.2) (layer "F.Cu") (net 10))
 (segment (start 139.48 102.64) (end 141.152 100.968) (width 0.2) (layer "F.Cu") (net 10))
 (segment (start 143.29 88.7926) (end 143.29 86.6613) (width 0.2) (layer "F.Cu") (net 10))
 (segment (start 150.754 73.4562) (end 150.754 61.975) (width 0.2) (layer "F.Cu") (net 10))
 (segment (start 139.286 110.454) (end 139.286 124.2465) (width 0.2) (layer "F.Cu") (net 13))
 (segment (start 139.286 124.2465) (end 139.2859 124.2466) (width 0.2) (layer "F.Cu") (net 13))
 (segment (start 139.286 124.2465) (end 139.286 127.165) (width 0.2) (layer "F.Cu") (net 13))
 (segment (start 147.1 102.64) (end 139.286 110.454) (width 0.2) (layer "F.Cu") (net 13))
 (segment (start 139.2859 124.2466) (end 139.2859 127.1651) (width 0.2) (layer "F.Cu") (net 13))
 (segment (start 145.348 106.932) (end 145.348 124.7315) (width 0.2) (layer "F.Cu") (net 14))
 (segment (start 149.64 102.64) (end 145.348 106.932) (width 0.2) (layer "F.Cu") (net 14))
 (segment (start 145.3481 124.7316) (end 145.3481 130.6651) (width 0.2) (layer "F.Cu") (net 14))
 (segment (start 145.348 124.7315) (end 145.3481 124.7316) (width 0.2) (layer "F.Cu") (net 14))
 (segment (start 145.348 124.7315) (end 145.348 130.665) (width 0.2) (layer "F.Cu") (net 14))
 (segment (start 205.75 94.5) (end 204.079 96.1709) (width 0.2) (layer "F.Cu") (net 7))
 (via (at 204.079 96.1709) (size 0.6) (drill 0.3) (layers "F.Cu" "B.Cu") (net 7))
 (segment (start 157.26 102.64) (end 163.729 96.1709) (width 0.2) (layer "B.Cu") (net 7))
 (segment (start 163.729 96.1709) (end 204.079 96.1709) (width 0.2) (layer "B.Cu") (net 7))
 (segment (start 205.75 101.5) (end 203.457 103.793) (width 0.2) (layer "F.Cu") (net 5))
 (segment (start 203.457 103.793) (end 201.858 103.793) (width 0.2) (layer "F.Cu") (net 5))
 (via (at 201.858 103.793) (size 0.6) (drill 0.3) (layers "F.Cu" "B.Cu") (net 5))
 (segment (start 201.858 103.793) (end 155.873 103.793) (width 0.2) (layer "B.Cu") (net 5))
 (segment (start 155.873 103.793) (end 154.72 102.64) (width 0.2) (layer "B.Cu") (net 5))
 (segment (start 158.53 113.53) (end 167.5 122.5) (width 0.2) (layer "F.Cu") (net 4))
 (segment (start 158.53 93.75) (end 158.53 113.53) (width 0.2) (layer "F.Cu") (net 4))
 (segment (start 152.18 87.4) (end 158.53 93.75) (width 0.2) (layer "F.Cu") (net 4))
 (segment (start 152.129 100.864) (end 153.45 102.185) (width 0.2) (layer "B.Cu") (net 3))
 (segment (start 150.91 88.67) (end 150.91 95.6793) (width 0.2) (layer "B.Cu") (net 3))
 (segment (start 152.129 96.8985) (end 152.129 100.864) (width 0.2) (layer "B.Cu") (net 3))
 (segment (start 150.91 95.6793) (end 152.129 96.8985) (width 0.2) (layer "B.Cu") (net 3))
 (segment (start 153.45 102.185) (end 153.45 110.99) (width 0.2) (layer "B.Cu") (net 3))
 (segment (start 153.45 110.99) (end 167.5 125.04) (width 0.2) (layer "B.Cu") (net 3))
 (segment (start 149.64 87.4) (end 150.91 88.67) (width 0.2) (layer "B.Cu") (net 3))
 (segment (start 148.379 112.935) (end 148.379 125.9215) (width 0.2) (layer "F.Cu") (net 15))
 (segment (start 148.3792 125.9217) (end 148.3792 132.4151) (width 0.2) (layer "F.Cu") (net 15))
 (segment (start 148.379 125.9215) (end 148.3792 125.9217) (width 0.2) (layer "F.Cu") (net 15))
 (segment (start 148.379 125.9215) (end 148.379 132.415) (width 0.2) (layer "F.Cu") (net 15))
 (segment (start 152.18 102.64) (end 148.379 106.441) (width 0.2) (layer "F.Cu") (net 15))
 (segment (start 148.379 112.934) (end 148.379 112.935) (width 0.2) (layer "F.Cu") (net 15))
 (segment (start 148.379 106.441) (end 148.379 112.934) (width 0.2) (layer "F.Cu") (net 15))
 (segment (start 207.368 86.2664) (end 201.311 80.2098) (width 0.2) (layer "F.Cu") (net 8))
 (segment (start 166.15 96.29) (end 159.8 102.64) (width 0.2) (layer "F.Cu") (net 8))
 (segment (start 207.368 89.3825) (end 207.368 86.2664) (width 0.2) (layer "F.Cu") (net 8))
 (segment (start 205.75 91) (end 207.368 89.3825) (width 0.2) (layer "F.Cu") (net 8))
 (segment (start 201.311 80.2098) (end 173.049 80.2098) (width 0.2) (layer "F.Cu") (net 8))
 (segment (start 173.049 80.2098) (end 166.15 87.1091) (width 0.2) (layer "F.Cu") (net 8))
 (segment (start 166.15 87.1091) (end 166.15 96.29) (width 0.2) (layer "F.Cu") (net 8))
 (segment (start 140.75 62.3953) (end 141.6609 61.4844) (width 0.2) (layer "F.Cu") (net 12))
 (segment (start 143.446 103.754) (end 139.012 103.754) (width 0.2) (layer "F.Cu") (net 12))
 (segment (start 139.012 103.754) (end 138.36 103.102) (width 0.2) (layer "F.Cu") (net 12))
 (segment (start 138.36 97.1551) (end 140.75 94.7653) (width 0.2) (layer "F.Cu") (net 12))
 (segment (start 138.36 103.102) (end 138.36 97.1551) (width 0.2) (layer "F.Cu") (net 12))
 (segment (start 140.75 94.7653) (end 140.75 62.3953) (width 0.2) (layer "F.Cu") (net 12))
 (segment (start 144.56 102.64) (end 143.446 103.754) (width 0.2) (layer "F.Cu") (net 12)))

